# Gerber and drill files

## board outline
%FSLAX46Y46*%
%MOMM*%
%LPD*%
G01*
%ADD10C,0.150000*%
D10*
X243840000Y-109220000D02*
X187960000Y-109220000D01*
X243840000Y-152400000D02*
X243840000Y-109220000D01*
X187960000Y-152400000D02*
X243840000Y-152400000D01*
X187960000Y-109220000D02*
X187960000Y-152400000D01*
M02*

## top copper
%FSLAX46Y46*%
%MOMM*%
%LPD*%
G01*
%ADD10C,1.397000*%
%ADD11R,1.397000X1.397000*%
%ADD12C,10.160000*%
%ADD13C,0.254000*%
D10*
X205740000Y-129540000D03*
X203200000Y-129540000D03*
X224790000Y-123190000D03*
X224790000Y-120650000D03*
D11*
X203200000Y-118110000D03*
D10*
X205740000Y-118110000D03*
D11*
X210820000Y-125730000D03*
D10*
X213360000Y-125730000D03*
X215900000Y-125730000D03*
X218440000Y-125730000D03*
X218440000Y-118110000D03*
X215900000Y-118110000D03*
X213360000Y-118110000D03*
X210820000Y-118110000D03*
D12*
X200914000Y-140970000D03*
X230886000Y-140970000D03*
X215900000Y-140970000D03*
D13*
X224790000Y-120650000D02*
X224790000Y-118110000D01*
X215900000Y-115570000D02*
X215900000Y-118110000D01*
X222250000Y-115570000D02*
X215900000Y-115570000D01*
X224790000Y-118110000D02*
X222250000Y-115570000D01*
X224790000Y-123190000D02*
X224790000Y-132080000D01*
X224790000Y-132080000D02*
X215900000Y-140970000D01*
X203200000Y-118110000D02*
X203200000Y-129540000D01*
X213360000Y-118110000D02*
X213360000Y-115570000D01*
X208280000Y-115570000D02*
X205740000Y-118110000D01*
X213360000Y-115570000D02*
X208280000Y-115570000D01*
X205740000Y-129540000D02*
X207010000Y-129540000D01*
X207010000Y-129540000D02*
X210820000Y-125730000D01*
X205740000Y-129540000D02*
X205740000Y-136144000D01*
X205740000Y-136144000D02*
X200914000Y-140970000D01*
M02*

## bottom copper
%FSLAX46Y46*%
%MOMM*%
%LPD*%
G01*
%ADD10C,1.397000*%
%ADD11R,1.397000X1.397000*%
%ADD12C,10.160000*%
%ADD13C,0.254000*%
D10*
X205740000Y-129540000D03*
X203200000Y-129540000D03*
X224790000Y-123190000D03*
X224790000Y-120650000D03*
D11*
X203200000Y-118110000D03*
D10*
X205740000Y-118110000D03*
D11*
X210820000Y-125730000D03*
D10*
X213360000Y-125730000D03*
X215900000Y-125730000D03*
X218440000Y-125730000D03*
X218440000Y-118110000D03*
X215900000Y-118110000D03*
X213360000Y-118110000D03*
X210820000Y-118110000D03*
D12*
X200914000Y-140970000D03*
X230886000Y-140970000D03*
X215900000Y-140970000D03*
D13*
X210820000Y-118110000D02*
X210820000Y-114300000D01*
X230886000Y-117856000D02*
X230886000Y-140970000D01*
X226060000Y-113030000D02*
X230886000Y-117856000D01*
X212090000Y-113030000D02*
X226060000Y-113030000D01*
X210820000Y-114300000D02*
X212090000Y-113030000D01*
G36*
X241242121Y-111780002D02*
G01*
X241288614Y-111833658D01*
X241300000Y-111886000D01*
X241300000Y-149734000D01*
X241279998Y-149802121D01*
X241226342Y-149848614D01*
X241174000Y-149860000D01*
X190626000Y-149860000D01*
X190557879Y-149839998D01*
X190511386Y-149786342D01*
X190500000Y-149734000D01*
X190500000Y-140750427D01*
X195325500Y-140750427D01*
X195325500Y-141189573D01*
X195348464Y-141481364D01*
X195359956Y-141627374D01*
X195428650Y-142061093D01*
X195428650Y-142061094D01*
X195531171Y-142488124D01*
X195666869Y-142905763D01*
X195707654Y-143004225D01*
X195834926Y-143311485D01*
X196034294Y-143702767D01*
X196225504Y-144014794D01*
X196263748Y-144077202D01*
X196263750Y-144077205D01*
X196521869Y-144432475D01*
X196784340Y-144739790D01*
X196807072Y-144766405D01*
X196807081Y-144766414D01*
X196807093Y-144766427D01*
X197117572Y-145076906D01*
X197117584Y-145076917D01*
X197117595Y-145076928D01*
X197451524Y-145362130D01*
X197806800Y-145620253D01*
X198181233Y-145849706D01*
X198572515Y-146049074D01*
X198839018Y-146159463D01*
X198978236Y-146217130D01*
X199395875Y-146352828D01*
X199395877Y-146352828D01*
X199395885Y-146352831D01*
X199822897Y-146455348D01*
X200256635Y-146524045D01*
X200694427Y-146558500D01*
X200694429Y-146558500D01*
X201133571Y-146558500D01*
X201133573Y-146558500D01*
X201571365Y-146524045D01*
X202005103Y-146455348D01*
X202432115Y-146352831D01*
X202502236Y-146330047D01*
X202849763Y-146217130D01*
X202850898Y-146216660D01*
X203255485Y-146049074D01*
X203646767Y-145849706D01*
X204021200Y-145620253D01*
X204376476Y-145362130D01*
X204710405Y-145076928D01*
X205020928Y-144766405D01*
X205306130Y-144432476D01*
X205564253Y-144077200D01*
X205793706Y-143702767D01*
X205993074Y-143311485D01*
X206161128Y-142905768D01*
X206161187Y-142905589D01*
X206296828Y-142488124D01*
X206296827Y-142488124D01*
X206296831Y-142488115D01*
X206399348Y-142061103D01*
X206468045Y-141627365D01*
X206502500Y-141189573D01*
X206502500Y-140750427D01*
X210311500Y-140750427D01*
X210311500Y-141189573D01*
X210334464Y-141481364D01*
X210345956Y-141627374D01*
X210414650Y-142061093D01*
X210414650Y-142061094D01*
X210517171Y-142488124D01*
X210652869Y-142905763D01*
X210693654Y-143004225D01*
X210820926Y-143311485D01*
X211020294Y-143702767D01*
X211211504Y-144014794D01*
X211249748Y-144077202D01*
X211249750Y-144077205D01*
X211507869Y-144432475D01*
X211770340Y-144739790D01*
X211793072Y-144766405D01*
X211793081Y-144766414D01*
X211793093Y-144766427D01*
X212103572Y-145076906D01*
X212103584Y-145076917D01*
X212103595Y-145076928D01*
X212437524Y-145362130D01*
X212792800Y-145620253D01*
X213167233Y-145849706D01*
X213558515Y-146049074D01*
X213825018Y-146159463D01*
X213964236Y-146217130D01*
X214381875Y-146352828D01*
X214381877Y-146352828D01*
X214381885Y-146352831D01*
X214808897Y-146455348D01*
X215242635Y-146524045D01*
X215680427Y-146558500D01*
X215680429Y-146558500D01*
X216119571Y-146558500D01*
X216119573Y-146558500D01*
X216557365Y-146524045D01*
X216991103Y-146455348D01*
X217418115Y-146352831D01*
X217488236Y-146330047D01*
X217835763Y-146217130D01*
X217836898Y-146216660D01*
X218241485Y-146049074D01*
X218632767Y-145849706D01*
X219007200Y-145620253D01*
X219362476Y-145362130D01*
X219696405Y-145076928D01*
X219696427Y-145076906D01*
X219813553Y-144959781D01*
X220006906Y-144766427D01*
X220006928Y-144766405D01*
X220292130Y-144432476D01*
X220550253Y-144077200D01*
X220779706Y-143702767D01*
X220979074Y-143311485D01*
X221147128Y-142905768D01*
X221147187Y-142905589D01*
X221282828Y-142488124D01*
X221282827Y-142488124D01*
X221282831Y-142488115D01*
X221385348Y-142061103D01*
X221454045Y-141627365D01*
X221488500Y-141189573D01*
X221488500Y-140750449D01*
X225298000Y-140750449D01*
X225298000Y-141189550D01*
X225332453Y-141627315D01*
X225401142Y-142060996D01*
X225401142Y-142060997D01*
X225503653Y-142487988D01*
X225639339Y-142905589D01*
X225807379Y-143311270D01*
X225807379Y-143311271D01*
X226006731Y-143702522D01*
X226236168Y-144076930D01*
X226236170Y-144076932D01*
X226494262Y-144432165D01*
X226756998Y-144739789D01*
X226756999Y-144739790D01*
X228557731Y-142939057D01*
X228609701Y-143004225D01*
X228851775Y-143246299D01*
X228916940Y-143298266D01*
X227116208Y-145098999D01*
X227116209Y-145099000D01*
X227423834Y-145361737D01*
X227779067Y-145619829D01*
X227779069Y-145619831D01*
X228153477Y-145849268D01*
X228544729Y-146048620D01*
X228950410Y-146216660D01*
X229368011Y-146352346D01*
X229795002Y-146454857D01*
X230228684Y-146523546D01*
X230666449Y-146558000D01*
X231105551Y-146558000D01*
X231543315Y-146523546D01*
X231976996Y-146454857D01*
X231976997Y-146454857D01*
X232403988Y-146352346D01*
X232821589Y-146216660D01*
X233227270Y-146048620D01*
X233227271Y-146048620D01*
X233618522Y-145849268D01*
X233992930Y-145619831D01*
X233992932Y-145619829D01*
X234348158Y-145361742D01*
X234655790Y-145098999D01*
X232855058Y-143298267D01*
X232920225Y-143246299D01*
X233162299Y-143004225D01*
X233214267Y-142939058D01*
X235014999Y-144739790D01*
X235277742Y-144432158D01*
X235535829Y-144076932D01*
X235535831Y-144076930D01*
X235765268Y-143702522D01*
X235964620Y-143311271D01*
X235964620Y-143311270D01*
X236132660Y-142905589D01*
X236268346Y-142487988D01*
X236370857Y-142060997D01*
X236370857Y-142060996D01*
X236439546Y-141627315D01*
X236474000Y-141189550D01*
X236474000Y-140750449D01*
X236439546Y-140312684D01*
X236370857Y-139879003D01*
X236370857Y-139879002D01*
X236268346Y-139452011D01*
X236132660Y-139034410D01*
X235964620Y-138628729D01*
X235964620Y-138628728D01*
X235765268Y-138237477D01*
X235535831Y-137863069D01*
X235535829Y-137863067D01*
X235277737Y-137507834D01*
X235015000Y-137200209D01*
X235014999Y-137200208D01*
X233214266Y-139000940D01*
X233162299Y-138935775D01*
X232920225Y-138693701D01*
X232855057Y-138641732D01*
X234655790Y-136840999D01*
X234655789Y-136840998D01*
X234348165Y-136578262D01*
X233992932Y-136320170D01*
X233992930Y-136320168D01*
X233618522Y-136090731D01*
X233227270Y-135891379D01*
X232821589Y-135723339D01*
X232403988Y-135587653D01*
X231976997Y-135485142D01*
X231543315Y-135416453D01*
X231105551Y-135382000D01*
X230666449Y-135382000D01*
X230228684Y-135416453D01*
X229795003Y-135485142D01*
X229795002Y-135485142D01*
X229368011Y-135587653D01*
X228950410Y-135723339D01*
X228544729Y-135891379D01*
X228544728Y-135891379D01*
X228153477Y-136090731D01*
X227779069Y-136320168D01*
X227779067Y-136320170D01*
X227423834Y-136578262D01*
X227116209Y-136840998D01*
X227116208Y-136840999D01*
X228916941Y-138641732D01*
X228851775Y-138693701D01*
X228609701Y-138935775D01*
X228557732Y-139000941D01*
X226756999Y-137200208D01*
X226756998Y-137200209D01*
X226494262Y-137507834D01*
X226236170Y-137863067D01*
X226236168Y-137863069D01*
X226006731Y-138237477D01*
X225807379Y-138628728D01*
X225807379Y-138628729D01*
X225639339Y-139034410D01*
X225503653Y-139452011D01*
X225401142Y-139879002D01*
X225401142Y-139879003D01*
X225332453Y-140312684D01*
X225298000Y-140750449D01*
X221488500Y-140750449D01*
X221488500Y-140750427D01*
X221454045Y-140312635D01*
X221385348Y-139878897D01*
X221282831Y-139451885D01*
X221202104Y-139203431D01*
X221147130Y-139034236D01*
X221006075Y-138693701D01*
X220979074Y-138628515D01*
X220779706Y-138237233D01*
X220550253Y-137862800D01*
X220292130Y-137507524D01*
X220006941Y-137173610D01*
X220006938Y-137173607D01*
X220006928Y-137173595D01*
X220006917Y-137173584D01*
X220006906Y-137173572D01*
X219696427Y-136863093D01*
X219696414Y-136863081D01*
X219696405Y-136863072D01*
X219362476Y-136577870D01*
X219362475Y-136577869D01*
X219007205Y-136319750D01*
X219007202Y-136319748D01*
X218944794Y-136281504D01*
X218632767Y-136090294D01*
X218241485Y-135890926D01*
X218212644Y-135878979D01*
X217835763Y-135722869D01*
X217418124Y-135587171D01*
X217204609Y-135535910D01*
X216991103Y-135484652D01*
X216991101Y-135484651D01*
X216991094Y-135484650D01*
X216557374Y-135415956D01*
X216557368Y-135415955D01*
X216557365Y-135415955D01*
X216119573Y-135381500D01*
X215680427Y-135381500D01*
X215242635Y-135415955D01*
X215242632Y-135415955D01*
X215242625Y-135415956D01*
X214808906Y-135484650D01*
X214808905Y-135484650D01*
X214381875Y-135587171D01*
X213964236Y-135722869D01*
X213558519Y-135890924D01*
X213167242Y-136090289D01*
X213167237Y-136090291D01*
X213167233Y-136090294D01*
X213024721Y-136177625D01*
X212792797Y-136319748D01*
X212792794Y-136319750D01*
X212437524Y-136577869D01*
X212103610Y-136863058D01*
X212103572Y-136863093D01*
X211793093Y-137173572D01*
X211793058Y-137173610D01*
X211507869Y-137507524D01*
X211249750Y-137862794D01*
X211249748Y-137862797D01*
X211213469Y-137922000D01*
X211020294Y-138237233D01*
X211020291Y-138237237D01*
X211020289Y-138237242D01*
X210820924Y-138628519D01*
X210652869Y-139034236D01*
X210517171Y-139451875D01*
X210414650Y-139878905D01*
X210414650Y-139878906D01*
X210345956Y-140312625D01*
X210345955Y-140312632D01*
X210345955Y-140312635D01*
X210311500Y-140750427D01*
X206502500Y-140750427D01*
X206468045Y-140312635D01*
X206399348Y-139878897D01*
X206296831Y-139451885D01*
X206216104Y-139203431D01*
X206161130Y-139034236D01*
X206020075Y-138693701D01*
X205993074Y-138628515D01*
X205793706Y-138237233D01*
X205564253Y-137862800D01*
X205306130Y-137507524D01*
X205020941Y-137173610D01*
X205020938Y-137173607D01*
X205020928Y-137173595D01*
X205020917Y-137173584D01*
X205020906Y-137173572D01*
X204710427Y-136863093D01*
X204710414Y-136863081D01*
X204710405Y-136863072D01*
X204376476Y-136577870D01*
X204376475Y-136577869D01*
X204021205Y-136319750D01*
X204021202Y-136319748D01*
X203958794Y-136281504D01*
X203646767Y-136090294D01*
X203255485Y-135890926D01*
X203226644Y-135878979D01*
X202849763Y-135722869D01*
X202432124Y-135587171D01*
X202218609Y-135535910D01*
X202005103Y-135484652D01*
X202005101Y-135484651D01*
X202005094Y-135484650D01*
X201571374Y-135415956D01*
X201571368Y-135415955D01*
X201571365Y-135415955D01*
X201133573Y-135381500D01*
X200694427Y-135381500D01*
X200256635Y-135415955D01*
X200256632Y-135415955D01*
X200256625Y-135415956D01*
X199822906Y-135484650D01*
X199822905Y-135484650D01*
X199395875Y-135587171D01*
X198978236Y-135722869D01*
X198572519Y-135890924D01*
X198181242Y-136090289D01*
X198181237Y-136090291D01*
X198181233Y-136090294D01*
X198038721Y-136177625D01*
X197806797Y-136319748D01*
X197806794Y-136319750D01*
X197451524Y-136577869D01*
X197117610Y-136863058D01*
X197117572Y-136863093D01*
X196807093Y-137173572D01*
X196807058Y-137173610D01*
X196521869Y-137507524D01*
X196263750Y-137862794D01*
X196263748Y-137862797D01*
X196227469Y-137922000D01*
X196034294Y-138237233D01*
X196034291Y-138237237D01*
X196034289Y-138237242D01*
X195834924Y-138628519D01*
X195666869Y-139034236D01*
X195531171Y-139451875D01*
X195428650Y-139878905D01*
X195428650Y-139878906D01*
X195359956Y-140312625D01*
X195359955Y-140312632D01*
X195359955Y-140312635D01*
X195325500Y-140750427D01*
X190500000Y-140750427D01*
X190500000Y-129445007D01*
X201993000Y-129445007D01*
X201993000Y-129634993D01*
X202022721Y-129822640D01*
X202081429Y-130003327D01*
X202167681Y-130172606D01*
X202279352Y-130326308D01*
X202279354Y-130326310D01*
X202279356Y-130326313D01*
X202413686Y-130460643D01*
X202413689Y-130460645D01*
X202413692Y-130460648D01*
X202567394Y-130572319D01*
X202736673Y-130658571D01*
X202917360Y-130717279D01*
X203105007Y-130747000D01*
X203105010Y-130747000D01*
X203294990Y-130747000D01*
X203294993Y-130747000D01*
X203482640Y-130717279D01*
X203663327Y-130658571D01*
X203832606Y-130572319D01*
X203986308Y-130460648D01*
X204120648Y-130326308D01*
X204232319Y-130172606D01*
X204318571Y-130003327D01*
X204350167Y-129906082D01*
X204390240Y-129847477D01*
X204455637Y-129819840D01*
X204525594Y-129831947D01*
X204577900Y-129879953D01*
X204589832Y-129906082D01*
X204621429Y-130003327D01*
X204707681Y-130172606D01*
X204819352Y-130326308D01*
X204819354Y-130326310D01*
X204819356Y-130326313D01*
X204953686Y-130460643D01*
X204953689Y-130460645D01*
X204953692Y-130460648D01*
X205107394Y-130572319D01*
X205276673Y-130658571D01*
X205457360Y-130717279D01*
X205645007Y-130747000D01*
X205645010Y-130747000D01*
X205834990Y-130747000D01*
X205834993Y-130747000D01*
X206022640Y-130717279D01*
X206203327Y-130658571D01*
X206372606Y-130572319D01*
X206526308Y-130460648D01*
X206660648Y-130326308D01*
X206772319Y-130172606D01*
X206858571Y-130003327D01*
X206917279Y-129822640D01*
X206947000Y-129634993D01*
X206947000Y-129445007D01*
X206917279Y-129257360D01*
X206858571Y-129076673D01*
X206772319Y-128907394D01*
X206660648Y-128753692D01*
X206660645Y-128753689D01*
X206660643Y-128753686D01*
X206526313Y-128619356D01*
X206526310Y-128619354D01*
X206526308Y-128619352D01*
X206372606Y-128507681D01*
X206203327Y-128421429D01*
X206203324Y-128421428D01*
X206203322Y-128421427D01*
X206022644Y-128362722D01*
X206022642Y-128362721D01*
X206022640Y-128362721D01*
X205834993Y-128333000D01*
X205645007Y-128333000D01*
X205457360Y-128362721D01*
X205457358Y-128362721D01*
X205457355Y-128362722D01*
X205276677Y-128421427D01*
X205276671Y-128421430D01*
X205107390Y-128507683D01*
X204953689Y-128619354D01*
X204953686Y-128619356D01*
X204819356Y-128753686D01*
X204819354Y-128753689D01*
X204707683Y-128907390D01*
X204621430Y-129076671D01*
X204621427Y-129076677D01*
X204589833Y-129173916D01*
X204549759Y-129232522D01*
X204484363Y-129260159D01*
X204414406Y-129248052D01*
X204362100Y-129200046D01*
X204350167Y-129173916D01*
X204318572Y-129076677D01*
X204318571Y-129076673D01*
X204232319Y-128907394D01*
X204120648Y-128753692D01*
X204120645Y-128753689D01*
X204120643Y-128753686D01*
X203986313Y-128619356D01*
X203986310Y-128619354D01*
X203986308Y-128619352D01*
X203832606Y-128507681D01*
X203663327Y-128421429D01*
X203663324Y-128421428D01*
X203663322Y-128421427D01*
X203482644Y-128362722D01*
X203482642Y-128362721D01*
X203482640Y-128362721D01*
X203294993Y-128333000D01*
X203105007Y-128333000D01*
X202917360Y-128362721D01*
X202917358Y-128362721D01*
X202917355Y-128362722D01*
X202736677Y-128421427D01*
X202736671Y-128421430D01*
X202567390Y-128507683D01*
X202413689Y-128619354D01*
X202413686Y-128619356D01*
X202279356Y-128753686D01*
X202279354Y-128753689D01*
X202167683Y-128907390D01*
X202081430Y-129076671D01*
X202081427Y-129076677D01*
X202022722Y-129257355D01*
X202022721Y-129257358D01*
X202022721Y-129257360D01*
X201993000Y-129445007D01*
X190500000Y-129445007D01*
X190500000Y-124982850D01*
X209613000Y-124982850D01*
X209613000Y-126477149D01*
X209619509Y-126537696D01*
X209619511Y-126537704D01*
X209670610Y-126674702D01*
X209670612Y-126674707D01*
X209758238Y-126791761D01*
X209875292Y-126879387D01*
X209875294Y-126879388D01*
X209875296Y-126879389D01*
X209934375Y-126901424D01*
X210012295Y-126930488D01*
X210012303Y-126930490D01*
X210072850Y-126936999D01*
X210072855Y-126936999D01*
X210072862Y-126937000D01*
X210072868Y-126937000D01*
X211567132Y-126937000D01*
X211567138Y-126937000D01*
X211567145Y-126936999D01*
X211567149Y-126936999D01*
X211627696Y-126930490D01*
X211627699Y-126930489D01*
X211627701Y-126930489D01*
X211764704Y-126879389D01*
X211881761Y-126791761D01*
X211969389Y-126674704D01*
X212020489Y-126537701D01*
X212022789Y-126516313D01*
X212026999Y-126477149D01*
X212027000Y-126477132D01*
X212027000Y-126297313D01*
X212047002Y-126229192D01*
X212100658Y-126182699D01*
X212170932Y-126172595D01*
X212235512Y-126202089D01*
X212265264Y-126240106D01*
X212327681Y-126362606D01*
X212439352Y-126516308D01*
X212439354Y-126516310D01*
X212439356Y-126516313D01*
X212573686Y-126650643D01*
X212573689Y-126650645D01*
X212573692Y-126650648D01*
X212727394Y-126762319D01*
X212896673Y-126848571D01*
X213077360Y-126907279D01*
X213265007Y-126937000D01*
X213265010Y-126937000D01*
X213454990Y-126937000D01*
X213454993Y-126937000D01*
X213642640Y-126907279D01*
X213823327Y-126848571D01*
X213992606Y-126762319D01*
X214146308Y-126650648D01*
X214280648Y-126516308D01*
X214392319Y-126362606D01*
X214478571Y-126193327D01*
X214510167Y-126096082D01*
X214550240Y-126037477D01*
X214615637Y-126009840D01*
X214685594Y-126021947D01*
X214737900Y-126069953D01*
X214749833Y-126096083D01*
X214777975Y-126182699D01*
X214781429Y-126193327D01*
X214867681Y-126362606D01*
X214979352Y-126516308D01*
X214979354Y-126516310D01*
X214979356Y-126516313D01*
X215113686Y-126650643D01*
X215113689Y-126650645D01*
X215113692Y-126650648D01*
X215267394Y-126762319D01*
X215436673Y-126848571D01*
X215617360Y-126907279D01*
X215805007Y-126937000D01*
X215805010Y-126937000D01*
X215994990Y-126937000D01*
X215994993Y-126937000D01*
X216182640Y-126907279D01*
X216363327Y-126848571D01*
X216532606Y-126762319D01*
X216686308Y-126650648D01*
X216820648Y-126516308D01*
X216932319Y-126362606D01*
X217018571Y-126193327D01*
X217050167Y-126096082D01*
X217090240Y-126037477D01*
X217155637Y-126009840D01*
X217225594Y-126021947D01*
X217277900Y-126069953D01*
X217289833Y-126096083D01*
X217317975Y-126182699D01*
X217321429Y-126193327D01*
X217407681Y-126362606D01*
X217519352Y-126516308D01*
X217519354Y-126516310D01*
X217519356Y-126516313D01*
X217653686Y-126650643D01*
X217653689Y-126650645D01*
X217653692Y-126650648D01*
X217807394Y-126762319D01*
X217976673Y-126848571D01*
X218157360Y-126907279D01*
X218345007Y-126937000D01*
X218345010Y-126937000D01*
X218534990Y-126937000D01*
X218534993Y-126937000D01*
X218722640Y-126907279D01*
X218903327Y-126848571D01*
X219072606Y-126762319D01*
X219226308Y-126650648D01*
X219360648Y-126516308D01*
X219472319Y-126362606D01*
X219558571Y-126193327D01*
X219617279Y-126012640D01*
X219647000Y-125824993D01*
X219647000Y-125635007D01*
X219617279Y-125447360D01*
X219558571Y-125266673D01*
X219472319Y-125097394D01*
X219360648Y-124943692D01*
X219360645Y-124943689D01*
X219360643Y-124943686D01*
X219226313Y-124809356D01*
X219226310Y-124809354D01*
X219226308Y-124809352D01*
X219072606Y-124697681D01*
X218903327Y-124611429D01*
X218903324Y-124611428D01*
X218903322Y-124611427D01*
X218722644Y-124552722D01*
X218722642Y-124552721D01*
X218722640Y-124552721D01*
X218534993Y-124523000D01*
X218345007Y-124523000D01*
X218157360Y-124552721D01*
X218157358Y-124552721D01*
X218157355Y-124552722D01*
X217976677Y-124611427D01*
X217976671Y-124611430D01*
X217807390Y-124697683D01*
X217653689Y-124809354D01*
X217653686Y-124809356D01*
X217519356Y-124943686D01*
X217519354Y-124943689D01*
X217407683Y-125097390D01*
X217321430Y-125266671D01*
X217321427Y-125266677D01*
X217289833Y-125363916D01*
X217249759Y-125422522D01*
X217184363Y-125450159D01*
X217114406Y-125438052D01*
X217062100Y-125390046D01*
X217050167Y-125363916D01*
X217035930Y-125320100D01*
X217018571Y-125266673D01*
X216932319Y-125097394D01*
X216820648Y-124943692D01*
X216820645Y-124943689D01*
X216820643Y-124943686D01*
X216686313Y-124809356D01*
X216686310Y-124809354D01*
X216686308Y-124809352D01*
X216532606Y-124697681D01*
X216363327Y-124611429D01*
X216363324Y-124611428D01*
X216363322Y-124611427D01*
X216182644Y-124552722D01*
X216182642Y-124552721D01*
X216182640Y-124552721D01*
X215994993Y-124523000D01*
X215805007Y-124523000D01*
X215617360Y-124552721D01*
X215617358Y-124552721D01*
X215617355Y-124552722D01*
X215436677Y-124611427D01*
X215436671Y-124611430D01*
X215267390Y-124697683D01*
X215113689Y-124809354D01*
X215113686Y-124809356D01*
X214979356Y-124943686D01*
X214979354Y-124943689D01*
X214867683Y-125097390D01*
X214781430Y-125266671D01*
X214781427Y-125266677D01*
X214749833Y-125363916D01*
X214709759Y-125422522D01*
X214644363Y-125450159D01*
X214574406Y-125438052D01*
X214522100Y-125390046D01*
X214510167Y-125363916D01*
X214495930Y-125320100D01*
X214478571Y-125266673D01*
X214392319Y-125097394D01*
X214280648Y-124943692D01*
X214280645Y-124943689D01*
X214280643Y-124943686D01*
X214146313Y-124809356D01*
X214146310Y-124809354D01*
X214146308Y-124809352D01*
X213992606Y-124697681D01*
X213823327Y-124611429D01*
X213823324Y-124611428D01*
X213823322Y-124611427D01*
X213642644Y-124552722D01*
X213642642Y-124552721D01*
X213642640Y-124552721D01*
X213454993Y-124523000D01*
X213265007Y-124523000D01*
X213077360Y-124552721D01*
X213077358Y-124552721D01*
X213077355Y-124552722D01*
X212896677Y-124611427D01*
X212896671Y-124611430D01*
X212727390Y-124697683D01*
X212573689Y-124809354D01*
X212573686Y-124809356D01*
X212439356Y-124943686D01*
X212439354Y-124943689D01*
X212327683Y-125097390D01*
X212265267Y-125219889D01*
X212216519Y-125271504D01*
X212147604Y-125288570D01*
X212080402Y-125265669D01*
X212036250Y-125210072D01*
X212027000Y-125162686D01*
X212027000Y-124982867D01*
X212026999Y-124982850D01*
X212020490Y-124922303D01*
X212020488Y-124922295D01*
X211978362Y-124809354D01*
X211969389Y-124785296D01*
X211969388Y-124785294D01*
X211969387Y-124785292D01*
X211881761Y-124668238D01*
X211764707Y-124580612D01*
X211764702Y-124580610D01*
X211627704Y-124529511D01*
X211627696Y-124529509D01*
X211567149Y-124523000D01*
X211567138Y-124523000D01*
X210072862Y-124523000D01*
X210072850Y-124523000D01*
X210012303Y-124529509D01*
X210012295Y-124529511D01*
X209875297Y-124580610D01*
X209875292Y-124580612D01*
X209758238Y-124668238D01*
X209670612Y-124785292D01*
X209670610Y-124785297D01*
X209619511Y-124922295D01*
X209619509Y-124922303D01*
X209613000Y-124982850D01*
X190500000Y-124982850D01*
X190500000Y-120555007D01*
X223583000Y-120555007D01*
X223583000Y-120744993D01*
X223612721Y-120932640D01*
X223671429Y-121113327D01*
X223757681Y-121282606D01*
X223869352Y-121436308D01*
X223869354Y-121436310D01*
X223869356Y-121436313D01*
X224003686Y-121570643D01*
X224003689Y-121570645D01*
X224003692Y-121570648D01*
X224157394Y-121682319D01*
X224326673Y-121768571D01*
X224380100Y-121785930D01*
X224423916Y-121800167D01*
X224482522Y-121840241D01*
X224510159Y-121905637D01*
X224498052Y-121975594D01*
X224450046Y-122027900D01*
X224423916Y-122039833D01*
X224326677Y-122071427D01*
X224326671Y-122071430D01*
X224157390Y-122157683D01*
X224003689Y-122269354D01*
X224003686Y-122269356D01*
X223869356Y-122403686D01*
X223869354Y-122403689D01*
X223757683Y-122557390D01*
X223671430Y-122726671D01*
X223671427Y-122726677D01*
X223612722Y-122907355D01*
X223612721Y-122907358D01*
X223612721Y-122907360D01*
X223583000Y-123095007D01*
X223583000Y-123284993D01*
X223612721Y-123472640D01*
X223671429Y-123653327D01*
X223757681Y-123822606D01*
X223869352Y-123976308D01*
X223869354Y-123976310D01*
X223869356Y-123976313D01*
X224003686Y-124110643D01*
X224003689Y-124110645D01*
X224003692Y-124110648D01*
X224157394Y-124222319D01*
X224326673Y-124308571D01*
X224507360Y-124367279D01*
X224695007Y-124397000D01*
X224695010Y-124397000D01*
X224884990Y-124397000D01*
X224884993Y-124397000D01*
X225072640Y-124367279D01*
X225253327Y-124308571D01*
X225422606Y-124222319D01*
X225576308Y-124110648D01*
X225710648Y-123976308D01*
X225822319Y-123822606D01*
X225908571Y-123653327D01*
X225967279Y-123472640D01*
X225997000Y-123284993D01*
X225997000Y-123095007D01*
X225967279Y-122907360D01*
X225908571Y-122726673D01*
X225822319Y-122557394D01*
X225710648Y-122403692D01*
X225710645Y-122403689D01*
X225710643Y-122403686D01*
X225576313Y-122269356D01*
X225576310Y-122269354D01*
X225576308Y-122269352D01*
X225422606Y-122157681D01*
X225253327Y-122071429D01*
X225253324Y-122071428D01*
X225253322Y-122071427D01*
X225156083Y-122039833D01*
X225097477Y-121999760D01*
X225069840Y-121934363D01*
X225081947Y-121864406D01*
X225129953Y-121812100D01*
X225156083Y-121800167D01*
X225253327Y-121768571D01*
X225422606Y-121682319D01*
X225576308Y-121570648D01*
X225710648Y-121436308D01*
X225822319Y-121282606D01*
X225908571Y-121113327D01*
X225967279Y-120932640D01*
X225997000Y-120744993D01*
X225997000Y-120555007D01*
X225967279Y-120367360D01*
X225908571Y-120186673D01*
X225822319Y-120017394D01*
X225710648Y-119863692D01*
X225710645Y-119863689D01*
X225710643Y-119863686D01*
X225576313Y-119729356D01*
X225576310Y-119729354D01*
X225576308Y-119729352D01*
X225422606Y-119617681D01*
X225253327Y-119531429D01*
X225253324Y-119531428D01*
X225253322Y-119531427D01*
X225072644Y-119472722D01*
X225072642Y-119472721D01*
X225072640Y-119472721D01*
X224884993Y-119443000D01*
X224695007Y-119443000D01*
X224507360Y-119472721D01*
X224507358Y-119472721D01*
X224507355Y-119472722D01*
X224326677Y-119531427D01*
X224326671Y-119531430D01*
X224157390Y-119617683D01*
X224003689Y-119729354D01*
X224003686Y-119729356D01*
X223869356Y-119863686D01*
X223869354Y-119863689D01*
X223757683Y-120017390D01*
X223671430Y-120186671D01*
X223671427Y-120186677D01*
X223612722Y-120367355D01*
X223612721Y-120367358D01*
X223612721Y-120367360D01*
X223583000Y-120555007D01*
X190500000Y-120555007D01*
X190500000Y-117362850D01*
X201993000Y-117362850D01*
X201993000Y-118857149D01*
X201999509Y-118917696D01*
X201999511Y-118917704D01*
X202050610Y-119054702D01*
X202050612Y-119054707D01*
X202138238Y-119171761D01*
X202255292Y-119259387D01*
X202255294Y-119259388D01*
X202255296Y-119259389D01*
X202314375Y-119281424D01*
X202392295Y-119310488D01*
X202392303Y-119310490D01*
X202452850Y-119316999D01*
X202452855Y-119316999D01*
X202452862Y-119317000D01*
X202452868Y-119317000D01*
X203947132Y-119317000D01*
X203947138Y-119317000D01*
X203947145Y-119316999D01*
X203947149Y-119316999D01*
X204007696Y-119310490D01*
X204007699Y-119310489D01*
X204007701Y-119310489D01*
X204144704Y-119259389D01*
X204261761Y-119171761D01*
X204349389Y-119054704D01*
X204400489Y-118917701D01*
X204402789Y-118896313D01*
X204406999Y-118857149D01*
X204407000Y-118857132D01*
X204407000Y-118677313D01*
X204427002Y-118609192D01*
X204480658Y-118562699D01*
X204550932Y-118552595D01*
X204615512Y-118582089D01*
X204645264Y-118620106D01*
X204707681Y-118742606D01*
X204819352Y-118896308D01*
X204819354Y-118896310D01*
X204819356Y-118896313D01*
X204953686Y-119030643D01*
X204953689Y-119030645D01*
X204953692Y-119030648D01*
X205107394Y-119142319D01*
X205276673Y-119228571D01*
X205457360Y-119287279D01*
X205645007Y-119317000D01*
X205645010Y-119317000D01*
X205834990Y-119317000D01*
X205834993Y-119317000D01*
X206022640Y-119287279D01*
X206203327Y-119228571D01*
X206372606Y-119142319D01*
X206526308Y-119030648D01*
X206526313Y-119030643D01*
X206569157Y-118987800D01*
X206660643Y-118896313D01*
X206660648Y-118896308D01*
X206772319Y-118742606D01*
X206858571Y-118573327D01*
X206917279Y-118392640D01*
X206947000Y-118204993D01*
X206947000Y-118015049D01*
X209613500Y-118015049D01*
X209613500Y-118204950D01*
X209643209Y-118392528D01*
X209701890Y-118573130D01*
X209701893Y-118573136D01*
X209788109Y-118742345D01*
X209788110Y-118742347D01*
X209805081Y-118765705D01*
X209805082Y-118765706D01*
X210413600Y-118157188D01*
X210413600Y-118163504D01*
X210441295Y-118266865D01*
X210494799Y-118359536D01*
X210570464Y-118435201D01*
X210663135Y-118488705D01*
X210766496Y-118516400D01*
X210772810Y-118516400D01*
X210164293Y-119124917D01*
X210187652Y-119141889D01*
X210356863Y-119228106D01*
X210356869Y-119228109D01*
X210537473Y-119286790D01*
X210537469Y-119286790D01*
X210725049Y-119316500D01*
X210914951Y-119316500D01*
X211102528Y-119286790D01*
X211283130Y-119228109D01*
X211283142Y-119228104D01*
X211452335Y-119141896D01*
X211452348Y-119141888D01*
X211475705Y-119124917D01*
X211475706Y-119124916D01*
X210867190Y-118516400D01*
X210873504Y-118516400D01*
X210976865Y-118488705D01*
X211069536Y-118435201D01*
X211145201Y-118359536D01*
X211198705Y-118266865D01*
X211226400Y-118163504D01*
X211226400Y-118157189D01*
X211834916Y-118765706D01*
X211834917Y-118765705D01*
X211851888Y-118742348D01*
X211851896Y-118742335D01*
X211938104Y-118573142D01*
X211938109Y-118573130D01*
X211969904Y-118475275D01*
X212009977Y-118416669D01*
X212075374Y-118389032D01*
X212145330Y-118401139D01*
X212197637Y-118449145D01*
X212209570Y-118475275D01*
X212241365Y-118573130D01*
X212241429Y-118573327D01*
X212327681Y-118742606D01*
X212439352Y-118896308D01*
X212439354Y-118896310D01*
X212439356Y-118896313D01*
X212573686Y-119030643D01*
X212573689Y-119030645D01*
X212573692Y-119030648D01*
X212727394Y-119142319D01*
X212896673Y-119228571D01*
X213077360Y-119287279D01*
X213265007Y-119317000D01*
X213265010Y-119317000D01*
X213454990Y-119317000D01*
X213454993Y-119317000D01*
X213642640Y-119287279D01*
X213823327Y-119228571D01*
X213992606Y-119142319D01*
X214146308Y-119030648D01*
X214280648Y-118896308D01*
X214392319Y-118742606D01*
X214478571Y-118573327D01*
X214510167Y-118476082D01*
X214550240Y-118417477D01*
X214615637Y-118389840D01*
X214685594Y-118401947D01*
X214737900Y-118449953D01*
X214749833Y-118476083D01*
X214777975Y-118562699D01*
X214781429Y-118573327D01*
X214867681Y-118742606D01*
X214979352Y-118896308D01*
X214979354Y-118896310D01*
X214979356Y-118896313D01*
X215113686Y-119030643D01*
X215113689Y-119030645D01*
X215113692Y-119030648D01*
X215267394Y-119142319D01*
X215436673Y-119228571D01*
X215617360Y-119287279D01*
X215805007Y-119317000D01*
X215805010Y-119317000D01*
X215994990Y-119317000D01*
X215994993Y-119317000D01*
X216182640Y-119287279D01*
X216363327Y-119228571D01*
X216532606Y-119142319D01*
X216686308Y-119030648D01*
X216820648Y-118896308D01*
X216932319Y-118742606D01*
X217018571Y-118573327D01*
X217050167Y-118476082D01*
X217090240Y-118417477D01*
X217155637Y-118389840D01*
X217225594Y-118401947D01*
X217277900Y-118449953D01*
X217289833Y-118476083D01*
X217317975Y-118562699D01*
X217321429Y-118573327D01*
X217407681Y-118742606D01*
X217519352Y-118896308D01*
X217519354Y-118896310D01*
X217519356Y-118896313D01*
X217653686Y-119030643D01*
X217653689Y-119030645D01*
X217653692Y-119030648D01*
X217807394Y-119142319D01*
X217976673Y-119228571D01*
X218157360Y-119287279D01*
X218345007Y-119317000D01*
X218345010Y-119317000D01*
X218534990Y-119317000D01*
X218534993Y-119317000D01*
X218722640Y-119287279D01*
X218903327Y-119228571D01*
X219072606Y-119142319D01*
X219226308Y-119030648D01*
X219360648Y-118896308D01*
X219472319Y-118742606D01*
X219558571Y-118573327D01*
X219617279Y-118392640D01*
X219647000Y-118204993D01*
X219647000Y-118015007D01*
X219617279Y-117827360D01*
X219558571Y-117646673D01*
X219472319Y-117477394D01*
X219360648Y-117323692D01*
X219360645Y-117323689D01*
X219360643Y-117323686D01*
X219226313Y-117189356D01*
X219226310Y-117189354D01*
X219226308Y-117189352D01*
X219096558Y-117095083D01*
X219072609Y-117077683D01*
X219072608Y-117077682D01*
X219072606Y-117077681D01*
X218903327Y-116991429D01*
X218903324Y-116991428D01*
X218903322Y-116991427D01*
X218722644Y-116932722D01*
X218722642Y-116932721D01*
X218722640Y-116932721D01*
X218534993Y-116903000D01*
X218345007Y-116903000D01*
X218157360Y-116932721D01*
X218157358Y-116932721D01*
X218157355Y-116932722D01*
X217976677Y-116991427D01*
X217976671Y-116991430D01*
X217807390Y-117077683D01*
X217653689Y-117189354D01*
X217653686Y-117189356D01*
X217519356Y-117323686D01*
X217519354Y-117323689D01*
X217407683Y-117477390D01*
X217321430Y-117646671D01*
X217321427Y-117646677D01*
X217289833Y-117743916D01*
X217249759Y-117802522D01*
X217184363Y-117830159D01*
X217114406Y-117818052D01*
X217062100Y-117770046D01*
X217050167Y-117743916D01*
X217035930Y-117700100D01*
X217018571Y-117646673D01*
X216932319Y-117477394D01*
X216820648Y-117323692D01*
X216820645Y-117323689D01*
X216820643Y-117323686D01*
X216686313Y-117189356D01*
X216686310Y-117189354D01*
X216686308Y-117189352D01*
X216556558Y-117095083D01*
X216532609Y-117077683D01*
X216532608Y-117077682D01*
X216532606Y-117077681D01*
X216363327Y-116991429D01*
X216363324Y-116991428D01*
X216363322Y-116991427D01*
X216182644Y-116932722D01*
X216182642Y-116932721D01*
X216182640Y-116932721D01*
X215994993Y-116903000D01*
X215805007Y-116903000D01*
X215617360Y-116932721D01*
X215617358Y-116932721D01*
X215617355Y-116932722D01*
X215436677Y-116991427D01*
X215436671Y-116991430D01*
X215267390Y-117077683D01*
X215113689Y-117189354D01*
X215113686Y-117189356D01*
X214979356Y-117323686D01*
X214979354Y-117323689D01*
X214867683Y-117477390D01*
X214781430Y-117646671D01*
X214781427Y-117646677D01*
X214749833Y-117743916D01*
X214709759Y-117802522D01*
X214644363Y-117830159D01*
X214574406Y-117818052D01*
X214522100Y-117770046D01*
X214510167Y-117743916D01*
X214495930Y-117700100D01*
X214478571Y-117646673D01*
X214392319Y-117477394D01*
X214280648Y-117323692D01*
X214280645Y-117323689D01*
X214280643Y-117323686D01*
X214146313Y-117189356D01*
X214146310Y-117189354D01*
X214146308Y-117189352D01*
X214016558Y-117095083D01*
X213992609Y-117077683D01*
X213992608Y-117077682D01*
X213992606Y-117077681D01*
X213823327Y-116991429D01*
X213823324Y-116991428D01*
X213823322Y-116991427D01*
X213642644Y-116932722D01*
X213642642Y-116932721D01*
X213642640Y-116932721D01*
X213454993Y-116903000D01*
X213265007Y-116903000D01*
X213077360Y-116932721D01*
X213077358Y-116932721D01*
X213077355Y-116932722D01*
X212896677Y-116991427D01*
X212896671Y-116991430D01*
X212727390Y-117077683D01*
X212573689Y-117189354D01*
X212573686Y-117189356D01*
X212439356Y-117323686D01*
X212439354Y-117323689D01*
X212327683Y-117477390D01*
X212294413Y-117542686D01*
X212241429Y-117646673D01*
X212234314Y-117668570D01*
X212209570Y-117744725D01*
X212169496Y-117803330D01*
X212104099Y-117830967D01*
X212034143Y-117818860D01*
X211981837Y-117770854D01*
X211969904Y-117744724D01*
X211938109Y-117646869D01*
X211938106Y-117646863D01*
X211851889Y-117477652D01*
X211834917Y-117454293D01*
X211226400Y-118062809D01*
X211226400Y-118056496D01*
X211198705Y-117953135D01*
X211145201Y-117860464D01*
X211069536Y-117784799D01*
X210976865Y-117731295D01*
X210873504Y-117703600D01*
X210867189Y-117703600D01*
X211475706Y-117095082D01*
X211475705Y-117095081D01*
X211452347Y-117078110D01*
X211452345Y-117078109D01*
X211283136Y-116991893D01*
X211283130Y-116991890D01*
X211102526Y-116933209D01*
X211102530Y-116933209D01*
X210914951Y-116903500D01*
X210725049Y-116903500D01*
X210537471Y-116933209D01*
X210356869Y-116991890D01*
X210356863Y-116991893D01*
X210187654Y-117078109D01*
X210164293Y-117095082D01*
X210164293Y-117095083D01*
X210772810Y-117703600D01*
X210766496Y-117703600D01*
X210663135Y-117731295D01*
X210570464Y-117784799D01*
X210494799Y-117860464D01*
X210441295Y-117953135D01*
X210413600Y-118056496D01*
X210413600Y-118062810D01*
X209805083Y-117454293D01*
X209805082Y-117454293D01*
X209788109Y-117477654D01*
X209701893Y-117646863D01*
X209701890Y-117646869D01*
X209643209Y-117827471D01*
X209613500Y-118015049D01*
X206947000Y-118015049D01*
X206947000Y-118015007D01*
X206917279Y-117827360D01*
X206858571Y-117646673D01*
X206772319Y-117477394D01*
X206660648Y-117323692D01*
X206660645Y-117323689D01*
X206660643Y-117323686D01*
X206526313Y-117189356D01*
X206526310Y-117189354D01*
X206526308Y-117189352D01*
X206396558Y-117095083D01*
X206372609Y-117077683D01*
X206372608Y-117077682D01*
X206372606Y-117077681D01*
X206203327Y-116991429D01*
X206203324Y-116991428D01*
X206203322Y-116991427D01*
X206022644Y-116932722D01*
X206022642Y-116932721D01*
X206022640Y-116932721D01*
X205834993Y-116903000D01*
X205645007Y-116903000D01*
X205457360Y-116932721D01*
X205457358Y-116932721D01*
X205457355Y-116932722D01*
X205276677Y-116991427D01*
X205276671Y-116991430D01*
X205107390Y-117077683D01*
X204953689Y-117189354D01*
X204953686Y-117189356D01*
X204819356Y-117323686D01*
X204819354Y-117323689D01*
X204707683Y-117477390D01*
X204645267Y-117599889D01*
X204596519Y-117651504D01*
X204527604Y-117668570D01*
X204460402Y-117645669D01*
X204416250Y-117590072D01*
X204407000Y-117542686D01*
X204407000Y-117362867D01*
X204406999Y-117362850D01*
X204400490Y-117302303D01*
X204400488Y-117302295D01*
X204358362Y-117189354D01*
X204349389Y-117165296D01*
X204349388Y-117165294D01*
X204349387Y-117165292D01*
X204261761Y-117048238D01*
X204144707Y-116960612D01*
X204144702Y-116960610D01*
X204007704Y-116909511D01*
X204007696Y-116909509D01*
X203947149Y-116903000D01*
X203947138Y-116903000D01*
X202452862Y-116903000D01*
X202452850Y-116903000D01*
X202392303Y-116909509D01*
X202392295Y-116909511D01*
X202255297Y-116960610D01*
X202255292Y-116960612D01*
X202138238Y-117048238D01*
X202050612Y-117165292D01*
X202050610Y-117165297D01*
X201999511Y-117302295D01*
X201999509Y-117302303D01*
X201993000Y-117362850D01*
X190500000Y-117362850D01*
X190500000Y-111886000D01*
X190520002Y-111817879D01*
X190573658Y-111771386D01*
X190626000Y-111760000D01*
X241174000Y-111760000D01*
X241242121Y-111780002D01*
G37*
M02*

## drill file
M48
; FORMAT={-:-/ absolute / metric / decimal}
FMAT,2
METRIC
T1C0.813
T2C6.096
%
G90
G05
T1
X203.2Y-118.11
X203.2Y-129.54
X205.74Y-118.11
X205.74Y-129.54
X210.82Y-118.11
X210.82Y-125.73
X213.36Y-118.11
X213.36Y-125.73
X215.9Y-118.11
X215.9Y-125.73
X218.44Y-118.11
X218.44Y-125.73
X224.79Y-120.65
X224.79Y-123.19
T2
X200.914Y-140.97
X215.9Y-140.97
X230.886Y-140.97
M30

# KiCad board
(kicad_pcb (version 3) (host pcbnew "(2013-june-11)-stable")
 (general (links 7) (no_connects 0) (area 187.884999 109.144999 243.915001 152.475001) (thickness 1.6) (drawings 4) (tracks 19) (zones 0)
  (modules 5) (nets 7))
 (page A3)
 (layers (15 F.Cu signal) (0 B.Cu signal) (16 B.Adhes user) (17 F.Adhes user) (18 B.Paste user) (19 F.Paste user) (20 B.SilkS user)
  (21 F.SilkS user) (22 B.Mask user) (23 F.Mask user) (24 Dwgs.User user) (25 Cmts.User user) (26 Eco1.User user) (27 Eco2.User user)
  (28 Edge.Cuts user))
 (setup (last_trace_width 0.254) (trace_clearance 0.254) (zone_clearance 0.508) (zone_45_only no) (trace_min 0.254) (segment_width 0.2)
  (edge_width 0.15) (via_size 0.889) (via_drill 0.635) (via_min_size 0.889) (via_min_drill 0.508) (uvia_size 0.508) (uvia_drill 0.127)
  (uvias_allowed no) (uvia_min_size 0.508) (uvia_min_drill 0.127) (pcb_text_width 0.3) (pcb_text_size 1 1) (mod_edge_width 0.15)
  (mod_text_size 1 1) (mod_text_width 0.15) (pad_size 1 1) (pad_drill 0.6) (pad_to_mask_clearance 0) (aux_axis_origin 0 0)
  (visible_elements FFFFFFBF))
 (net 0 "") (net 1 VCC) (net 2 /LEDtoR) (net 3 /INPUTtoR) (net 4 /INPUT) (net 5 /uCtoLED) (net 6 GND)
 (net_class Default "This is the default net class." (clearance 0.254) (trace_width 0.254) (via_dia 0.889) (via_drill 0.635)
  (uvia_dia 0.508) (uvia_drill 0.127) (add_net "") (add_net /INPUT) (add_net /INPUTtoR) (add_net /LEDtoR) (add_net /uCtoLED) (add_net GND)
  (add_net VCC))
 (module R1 (layer F.Cu) (at 204.47 129.54 180) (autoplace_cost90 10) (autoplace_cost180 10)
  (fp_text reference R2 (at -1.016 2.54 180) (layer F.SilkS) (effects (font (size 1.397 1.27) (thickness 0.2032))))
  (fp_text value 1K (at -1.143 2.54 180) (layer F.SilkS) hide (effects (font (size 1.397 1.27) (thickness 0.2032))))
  (pad 1 thru_hole circle (at -1.27 0 180) (size 1.397 1.397) (drill 0.8128) (layers *.Cu *.Mask F.SilkS) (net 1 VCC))
  (pad 2 thru_hole circle (at 1.27 0 180) (size 1.397 1.397) (drill 0.8128) (layers *.Cu *.Mask F.SilkS) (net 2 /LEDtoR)))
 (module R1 (layer F.Cu) (at 224.79 121.92 90) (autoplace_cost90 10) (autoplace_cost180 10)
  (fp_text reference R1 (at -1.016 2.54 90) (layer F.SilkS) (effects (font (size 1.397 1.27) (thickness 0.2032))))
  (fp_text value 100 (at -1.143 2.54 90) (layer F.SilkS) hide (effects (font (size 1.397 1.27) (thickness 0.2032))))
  (pad 1 thru_hole circle (at -1.27 0 90) (size 1.397 1.397) (drill 0.8128) (layers *.Cu *.Mask F.SilkS) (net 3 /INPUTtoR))
  (pad 2 thru_hole circle (at 1.27 0 90) (size 1.397 1.397) (drill 0.8128) (layers *.Cu *.Mask F.SilkS) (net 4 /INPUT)))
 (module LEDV (layer F.Cu) (at 204.47 118.11)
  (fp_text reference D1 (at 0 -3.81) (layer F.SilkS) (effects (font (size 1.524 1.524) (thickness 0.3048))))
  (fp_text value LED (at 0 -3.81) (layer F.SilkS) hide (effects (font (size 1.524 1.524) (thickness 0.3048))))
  (pad 1 thru_hole rect (at -1.27 0) (size 1.397 1.397) (drill 0.8128) (layers *.Cu *.Mask F.SilkS) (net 2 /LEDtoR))
  (pad 2 thru_hole circle (at 1.27 0) (size 1.397 1.397) (drill 0.8128) (layers *.Cu *.Mask F.SilkS) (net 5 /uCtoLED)))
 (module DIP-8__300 (layer F.Cu) (at 214.63 121.92)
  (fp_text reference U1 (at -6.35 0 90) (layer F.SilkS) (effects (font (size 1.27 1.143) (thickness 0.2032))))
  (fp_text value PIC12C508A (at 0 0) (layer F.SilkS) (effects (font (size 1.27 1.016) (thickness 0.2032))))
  (pad 1 thru_hole rect (at -3.81 3.81) (size 1.397 1.397) (drill 0.8128) (layers *.Cu *.Mask F.SilkS) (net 1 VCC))
  (pad 2 thru_hole circle (at -1.27 3.81) (size 1.397 1.397) (drill 0.8128) (layers *.Cu *.Mask F.SilkS))
  (pad 3 thru_hole circle (at 1.27 3.81) (size 1.397 1.397) (drill 0.8128) (layers *.Cu *.Mask F.SilkS))
  (pad 4 thru_hole circle (at 3.81 3.81) (size 1.397 1.397) (drill 0.8128) (layers *.Cu *.Mask F.SilkS))
  (pad 5 thru_hole circle (at 3.81 -3.81) (size 1.397 1.397) (drill 0.8128) (layers *.Cu *.Mask F.SilkS))
  (pad 6 thru_hole circle (at 1.27 -3.81) (size 1.397 1.397) (drill 0.8128) (layers *.Cu *.Mask F.SilkS) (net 4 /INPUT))
  (pad 7 thru_hole circle (at -1.27 -3.81) (size 1.397 1.397) (drill 0.8128) (layers *.Cu *.Mask F.SilkS) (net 5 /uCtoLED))
  (pad 8 thru_hole circle (at -3.81 -3.81) (size 1.397 1.397) (drill 0.8128) (layers *.Cu *.Mask F.SilkS) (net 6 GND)))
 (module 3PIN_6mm (layer F.Cu) (at 215.9 140.97)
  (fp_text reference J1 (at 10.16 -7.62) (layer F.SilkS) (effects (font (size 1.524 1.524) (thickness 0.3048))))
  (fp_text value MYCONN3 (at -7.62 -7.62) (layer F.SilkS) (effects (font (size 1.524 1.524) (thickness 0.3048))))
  (pad 1 thru_hole circle (at -14.986 0) (size 10.16 10.16) (drill 6.096) (layers *.Cu *.Mask F.SilkS) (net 1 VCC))
  (pad 3 thru_hole circle (at 14.986 0) (size 10.16 10.16) (drill 6.096) (layers *.Cu *.Mask F.SilkS) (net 6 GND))
  (pad 2 thru_hole circle (at 0 0) (size 10.16 10.16) (drill 6.096) (layers *.Cu *.Mask F.SilkS) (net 3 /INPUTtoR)))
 (gr_line (start 243.84 109.22) (end 187.96 109.22) (angle 90) (layer Edge.Cuts) (width 0.15))
 (gr_line (start 243.84 152.4) (end 243.84 109.22) (angle 90) (layer Edge.Cuts) (width 0.15))
 (gr_line (start 187.96 152.4) (end 243.84 152.4) (angle 90) (layer Edge.Cuts) (width 0.15))
 (gr_line (start 187.96 109.22) (end 187.96 152.4) (angle 90) (layer Edge.Cuts) (width 0.15))
 (segment (start 224.79 120.65) (end 224.79 118.11) (width 0.254) (layer F.Cu) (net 4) (status 400000))
 (segment (start 215.9 115.57) (end 215.9 118.11) (width 0.254) (layer F.Cu) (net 4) (status 800000))
 (segment (start 222.25 115.57) (end 215.9 115.57) (width 0.254) (layer F.Cu) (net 4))
 (segment (start 224.79 118.11) (end 222.25 115.57) (width 0.254) (layer F.Cu) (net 4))
 (segment (start 224.79 123.19) (end 224.79 132.08) (width 0.254) (layer F.Cu) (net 3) (status 400000))
 (segment (start 224.79 132.08) (end 215.9 140.97) (width 0.254) (layer F.Cu) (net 3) (status 800000))
 (segment (start 203.2 118.11) (end 203.2 129.54) (width 0.254) (layer F.Cu) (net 2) (status C00000))
 (segment (start 213.36 118.11) (end 213.36 115.57) (width 0.254) (layer F.Cu) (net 5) (status 400000))
 (segment (start 208.28 115.57) (end 205.74 118.11) (width 0.254) (layer F.Cu) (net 5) (status 800000))
 (segment (start 213.36 115.57) (end 208.28 115.57) (width 0.254) (layer F.Cu) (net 5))
 (segment (start 210.82 118.11) (end 210.82 114.3) (width 0.254) (layer B.Cu) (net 6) (status 400000))
 (segment (start 230.886 117.856) (end 230.886 140.97) (width 0.254) (layer B.Cu) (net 6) (status 800000))
 (segment (start 226.06 113.03) (end 230.886 117.856) (width 0.254) (layer B.Cu) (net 6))
 (segment (start 212.09 113.03) (end 226.06 113.03) (width 0.254) (layer B.Cu) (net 6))
 (segment (start 210.82 114.3) (end 212.09 113.03) (width 0.254) (layer B.Cu) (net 6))
 (segment (start 205.74 129.54) (end 207.01 129.54) (width 0.254) (layer F.Cu) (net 1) (status 400000))
 (segment (start 207.01 129.54) (end 210.82 125.73) (width 0.254) (layer F.Cu) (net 1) (status 800000))
 (segment (start 205.74 129.54) (end 205.74 136.144) (width 0.254) (layer F.Cu) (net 1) (status 400000))
 (segment (start 205.74 136.144) (end 200.914 140.97) (width 0.254) (layer F.Cu) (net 1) (status 800000))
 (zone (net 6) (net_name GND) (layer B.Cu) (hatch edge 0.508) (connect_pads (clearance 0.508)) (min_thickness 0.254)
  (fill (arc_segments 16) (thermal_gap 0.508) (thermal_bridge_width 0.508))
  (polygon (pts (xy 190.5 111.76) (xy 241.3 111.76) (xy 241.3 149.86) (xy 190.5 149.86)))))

